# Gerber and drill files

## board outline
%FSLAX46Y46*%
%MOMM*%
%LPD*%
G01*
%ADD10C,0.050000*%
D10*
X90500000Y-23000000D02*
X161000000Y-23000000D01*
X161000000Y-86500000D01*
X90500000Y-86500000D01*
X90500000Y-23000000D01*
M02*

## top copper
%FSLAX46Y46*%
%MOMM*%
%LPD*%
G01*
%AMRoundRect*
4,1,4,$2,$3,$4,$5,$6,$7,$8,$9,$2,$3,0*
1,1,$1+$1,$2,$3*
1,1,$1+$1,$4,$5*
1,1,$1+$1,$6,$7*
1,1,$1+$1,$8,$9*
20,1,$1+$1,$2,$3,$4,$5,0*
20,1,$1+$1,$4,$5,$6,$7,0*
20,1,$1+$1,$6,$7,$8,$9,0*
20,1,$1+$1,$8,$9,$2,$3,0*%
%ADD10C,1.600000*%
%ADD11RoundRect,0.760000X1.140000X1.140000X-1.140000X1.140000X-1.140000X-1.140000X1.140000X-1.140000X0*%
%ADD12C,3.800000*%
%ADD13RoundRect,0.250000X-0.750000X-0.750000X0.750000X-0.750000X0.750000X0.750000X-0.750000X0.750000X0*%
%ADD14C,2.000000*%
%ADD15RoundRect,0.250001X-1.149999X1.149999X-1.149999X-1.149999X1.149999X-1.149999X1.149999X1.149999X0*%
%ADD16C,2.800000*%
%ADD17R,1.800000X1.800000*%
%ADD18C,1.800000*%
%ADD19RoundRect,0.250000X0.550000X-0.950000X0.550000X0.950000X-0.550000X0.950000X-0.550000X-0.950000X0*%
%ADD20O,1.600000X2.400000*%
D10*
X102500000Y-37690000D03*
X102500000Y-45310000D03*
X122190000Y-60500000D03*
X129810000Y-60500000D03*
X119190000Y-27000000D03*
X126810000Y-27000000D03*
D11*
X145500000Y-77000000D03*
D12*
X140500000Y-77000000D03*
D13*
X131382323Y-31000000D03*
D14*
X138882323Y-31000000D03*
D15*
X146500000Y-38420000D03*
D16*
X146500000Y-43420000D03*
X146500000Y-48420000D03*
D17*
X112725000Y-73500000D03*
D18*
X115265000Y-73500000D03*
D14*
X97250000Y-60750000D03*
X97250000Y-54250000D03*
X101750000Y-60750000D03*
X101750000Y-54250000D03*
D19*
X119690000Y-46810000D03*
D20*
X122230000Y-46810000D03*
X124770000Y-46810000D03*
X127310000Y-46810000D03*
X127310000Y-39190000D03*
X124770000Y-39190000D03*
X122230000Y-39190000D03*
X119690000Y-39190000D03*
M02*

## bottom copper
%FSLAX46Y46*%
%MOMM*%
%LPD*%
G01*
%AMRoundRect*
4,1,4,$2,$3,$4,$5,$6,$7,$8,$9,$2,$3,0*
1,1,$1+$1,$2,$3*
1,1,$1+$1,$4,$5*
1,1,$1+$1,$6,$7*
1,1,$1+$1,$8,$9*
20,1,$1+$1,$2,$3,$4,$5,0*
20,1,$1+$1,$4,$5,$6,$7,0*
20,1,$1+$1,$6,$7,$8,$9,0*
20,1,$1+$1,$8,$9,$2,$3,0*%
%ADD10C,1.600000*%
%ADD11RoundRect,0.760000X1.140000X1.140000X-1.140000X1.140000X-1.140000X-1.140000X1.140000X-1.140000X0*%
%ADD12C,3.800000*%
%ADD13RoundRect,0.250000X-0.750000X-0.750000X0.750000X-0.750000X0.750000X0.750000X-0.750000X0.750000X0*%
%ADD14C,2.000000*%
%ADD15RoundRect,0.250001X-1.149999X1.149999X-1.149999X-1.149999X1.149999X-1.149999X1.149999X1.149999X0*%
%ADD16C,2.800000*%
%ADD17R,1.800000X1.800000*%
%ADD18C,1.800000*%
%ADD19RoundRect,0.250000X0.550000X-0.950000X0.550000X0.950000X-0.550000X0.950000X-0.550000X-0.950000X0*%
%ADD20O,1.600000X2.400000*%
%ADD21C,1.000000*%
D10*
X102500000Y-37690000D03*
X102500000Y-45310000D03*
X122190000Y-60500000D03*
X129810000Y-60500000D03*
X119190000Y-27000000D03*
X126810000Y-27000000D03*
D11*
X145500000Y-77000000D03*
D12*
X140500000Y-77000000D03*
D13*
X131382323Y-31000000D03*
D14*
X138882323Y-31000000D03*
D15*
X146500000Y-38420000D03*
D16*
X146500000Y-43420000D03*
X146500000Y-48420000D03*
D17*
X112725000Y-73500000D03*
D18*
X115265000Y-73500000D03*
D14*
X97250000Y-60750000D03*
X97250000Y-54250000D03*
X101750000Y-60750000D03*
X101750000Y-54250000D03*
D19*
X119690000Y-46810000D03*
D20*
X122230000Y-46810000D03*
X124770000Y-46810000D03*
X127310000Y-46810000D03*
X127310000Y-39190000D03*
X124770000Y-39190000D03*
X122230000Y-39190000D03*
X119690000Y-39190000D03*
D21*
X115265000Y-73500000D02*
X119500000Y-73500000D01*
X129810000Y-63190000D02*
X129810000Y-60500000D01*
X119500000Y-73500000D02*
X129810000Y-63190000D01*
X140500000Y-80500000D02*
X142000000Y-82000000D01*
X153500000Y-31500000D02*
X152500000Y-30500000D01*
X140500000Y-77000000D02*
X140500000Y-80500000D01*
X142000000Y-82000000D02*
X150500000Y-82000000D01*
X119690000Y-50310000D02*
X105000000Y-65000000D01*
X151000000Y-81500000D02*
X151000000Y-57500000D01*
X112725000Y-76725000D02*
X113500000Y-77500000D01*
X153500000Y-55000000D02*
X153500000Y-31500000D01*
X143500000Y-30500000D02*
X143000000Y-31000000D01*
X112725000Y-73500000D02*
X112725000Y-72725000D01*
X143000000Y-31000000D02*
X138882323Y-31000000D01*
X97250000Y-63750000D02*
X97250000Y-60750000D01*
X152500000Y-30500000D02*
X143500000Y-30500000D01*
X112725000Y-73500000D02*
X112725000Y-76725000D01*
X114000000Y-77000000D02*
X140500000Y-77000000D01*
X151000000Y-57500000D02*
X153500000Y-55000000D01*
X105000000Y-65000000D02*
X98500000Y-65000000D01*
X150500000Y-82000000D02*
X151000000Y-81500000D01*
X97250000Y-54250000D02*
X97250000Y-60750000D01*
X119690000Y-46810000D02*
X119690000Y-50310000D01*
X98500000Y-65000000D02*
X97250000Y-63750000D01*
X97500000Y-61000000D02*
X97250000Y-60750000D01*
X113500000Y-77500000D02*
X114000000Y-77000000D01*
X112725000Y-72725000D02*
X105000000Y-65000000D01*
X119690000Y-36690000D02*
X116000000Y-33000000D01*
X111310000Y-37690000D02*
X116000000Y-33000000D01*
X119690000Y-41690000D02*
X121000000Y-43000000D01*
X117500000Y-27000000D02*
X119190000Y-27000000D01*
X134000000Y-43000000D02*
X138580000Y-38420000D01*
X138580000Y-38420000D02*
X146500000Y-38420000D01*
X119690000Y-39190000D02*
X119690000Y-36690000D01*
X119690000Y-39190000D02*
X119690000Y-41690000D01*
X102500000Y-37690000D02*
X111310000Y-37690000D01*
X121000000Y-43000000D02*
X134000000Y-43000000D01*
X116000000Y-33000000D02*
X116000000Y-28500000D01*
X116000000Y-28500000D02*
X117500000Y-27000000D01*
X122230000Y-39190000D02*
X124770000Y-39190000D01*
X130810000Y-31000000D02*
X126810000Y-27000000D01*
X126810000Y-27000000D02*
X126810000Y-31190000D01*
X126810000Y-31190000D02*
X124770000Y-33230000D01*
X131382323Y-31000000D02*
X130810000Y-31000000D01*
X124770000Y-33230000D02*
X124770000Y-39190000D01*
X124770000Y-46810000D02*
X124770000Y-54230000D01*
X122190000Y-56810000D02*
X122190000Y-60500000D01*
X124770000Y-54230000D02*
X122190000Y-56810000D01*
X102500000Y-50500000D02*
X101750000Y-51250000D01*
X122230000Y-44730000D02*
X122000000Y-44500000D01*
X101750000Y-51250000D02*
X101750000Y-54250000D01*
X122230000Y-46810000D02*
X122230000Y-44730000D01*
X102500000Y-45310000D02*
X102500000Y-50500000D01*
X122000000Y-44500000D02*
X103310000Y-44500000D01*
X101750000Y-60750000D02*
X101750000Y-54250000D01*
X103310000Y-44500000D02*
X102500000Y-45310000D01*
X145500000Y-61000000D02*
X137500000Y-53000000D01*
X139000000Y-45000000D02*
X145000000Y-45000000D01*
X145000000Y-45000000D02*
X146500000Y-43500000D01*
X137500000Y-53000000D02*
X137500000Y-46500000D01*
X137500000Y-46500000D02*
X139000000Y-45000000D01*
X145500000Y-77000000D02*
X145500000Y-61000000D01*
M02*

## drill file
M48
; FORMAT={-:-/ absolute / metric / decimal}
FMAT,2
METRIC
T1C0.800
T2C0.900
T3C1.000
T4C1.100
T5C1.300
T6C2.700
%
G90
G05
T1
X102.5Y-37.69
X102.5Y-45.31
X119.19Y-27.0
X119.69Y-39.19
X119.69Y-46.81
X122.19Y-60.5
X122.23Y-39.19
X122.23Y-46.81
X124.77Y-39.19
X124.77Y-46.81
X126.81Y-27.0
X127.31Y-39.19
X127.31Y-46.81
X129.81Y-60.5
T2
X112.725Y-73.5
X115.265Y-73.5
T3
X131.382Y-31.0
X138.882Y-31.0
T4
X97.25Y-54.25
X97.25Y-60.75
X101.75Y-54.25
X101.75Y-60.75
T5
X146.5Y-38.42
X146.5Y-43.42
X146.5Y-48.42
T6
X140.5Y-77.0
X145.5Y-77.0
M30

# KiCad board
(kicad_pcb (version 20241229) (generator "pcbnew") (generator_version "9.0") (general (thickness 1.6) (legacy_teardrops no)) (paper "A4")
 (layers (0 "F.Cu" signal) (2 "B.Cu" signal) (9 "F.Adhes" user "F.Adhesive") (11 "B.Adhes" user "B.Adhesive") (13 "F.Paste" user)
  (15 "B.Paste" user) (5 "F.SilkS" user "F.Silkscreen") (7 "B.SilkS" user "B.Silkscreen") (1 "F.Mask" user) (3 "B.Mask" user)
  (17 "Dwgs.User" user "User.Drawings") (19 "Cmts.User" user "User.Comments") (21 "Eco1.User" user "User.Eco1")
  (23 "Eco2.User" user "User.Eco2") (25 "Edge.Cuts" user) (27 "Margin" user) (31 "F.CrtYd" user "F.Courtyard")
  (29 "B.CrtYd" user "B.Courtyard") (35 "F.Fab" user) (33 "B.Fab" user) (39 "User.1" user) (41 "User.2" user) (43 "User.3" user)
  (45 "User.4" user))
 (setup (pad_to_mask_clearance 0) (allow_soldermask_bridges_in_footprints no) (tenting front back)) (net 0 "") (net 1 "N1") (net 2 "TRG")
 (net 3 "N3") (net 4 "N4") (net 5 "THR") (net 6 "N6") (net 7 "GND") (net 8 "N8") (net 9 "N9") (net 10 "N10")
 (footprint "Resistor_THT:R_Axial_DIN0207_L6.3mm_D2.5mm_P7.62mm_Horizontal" (layer "F.Cu") (at 102.5 37.69 -90)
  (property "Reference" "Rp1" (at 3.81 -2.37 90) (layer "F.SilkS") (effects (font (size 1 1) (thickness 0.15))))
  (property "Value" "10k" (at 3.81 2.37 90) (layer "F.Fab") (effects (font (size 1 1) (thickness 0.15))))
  (pad "1" thru_hole circle (at 0 0 270) (size 1.6 1.6) (drill 0.8) (layers "*.Cu" "*.Mask") (remove_unused_layers no) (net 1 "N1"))
  (pad "2" thru_hole circle (at 7.62 0 270) (size 1.6 1.6) (drill 0.8) (layers "*.Cu" "*.Mask") (remove_unused_layers no) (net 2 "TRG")))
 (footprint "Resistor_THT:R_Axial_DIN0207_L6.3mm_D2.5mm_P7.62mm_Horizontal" (layer "F.Cu") (at 122.19 60.5)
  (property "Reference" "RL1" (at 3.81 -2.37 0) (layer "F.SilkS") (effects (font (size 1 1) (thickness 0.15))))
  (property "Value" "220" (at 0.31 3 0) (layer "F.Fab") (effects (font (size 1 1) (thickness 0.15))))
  (pad "1" thru_hole circle (at 0 0) (size 1.6 1.6) (drill 0.8) (layers "*.Cu" "*.Mask") (remove_unused_layers no) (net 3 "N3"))
  (pad "2" thru_hole circle (at 7.62 0) (size 1.6 1.6) (drill 0.8) (layers "*.Cu" "*.Mask") (remove_unused_layers no) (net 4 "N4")))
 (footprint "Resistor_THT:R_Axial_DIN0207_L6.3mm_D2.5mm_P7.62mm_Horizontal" (layer "F.Cu") (at 119.19 27)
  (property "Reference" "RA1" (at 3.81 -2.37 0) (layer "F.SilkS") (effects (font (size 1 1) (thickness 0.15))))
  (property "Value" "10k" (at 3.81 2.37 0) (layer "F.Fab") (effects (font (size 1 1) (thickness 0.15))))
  (pad "1" thru_hole circle (at 0 0) (size 1.6 1.6) (drill 0.8) (layers "*.Cu" "*.Mask") (remove_unused_layers no) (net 1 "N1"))
  (pad "2" thru_hole circle (at 7.62 0) (size 1.6 1.6) (drill 0.8) (layers "*.Cu" "*.Mask") (remove_unused_layers no) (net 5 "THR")))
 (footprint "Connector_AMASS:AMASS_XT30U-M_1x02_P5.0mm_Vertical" (layer "F.Cu") (at 145.5 77 180)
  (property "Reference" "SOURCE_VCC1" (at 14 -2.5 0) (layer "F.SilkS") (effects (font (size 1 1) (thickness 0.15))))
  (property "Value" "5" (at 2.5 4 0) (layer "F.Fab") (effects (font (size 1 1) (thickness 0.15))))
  (pad "1" thru_hole roundrect (at 0 0 180) (size 3.8 3.8) (drill 2.7) (layers "*.Cu" "*.Mask") (remove_unused_layers no)
   (roundrect_rratio 0.2) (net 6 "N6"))
  (pad "2" thru_hole circle (at 5 0 180) (size 3.8 3.8) (drill 2.7) (layers "*.Cu" "*.Mask") (remove_unused_layers no) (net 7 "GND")))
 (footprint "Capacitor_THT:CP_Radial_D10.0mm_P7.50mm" (layer "F.Cu") (at 131.382323 31)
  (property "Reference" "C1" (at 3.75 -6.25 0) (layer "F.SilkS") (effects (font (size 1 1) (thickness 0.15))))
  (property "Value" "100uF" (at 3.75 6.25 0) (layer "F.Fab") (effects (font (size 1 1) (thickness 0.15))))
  (pad "1" thru_hole roundrect (at 0 0) (size 2 2) (drill 1) (layers "*.Cu" "*.Mask") (remove_unused_layers no) (roundrect_rratio 0.125)
   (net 5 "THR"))
  (pad "2" thru_hole circle (at 7.5 0) (size 2 2) (drill 1) (layers "*.Cu" "*.Mask") (remove_unused_layers no) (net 7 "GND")))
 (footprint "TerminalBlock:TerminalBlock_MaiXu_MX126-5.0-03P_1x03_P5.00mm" (layer "F.Cu") (at 146.5 38.42 -90)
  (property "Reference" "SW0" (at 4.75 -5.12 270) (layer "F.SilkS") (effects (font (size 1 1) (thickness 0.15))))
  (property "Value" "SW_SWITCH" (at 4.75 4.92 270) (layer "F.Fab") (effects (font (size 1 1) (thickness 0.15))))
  (pad "1" thru_hole roundrect (at 0 0 270) (size 2.8 2.8) (drill 1.3) (layers "*.Cu" "*.Mask") (remove_unused_layers no)
   (roundrect_rratio 0.089286) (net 1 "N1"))
  (pad "2" thru_hole circle (at 5 0 270) (size 2.8 2.8) (drill 1.3) (layers "*.Cu" "*.Mask") (remove_unused_layers no) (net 6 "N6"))
  (pad "3" thru_hole circle (at 10 0 270) (size 2.8 2.8) (drill 1.3) (layers "*.Cu" "*.Mask") (remove_unused_layers no) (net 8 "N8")))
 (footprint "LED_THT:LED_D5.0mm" (layer "F.Cu") (at 112.725 73.5)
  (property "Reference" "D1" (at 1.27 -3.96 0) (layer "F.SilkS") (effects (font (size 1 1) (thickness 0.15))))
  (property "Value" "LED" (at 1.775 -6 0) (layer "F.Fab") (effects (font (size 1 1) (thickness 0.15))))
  (pad "1" thru_hole rect (at 0 0) (size 1.8 1.8) (drill 0.9) (layers "*.Cu" "*.Mask") (remove_unused_layers no) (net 7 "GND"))
  (pad "2" thru_hole circle (at 2.54 0) (size 1.8 1.8) (drill 0.9) (layers "*.Cu" "*.Mask") (remove_unused_layers no) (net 4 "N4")))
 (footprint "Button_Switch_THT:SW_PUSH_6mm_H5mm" (layer "F.Cu") (at 97.25 60.75 90)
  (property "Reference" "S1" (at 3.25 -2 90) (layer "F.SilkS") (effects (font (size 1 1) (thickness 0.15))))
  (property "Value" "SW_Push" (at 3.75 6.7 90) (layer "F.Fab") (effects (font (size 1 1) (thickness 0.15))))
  (pad "1" thru_hole circle (at 0 0 180) (size 2 2) (drill 1.1) (layers "*.Cu" "*.Mask") (remove_unused_layers no) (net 7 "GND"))
  (pad "1" thru_hole circle (at 6.5 0 180) (size 2 2) (drill 1.1) (layers "*.Cu" "*.Mask") (remove_unused_layers no) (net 7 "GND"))
  (pad "2" thru_hole circle (at 0 4.5 180) (size 2 2) (drill 1.1) (layers "*.Cu" "*.Mask") (remove_unused_layers no) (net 2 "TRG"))
  (pad "2" thru_hole circle (at 6.5 4.5 180) (size 2 2) (drill 1.1) (layers "*.Cu" "*.Mask") (remove_unused_layers no) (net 2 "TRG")))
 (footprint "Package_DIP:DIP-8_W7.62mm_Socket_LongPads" (layer "F.Cu") (at 119.69 46.81 90)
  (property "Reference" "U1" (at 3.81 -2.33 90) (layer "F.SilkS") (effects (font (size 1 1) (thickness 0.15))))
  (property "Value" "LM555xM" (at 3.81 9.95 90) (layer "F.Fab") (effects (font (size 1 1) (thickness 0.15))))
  (pad "1" thru_hole roundrect (at 0 0 90) (size 2.4 1.6) (drill 0.8) (layers "*.Cu" "*.Mask") (remove_unused_layers no)
   (roundrect_rratio 0.15625) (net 7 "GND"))
  (pad "2" thru_hole oval (at 0 2.54 90) (size 2.4 1.6) (drill 0.8) (layers "*.Cu" "*.Mask") (remove_unused_layers no) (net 2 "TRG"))
  (pad "3" thru_hole oval (at 0 5.08 90) (size 2.4 1.6) (drill 0.8) (layers "*.Cu" "*.Mask") (remove_unused_layers no) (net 3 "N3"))
  (pad "4" thru_hole oval (at 0 7.62 90) (size 2.4 1.6) (drill 0.8) (layers "*.Cu" "*.Mask") (remove_unused_layers no) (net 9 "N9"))
  (pad "5" thru_hole oval (at 7.62 7.62 90) (size 2.4 1.6) (drill 0.8) (layers "*.Cu" "*.Mask") (remove_unused_layers no) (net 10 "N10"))
  (pad "6" thru_hole oval (at 7.62 5.08 90) (size 2.4 1.6) (drill 0.8) (layers "*.Cu" "*.Mask") (remove_unused_layers no) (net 5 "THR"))
  (pad "7" thru_hole oval (at 7.62 2.54 90) (size 2.4 1.6) (drill 0.8) (layers "*.Cu" "*.Mask") (remove_unused_layers no) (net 5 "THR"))
  (pad "8" thru_hole oval (at 7.62 0 90) (size 2.4 1.6) (drill 0.8) (layers "*.Cu" "*.Mask") (remove_unused_layers no) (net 1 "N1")))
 (gr_rect (start 90.5 23) (end 161 86.5) (stroke (width 0.05) (type default)) (fill no) (layer "Edge.Cuts"))
 (segment (start 115.265 73.5) (end 119.5 73.5) (width 1) (layer "B.Cu") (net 4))
 (segment (start 129.81 63.19) (end 129.81 60.5) (width 1) (layer "B.Cu") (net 4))
 (segment (start 119.5 73.5) (end 129.81 63.19) (width 1) (layer "B.Cu") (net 4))
 (segment (start 140.5 80.5) (end 142 82) (width 1) (layer "B.Cu") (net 7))
 (segment (start 153.5 31.5) (end 152.5 30.5) (width 1) (layer "B.Cu") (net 7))
 (segment (start 140.5 77) (end 140.5 80.5) (width 1) (layer "B.Cu") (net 7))
 (segment (start 142 82) (end 150.5 82) (width 1) (layer "B.Cu") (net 7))
 (segment (start 119.69 50.31) (end 105 65) (width 1) (layer "B.Cu") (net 7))
 (segment (start 151 81.5) (end 151 57.5) (width 1) (layer "B.Cu") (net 7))
 (segment (start 112.725 76.725) (end 113.5 77.5) (width 1) (layer "B.Cu") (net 7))
 (segment (start 153.5 55) (end 153.5 31.5) (width 1) (layer "B.Cu") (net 7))
 (segment (start 143.5 30.5) (end 143 31) (width 1) (layer "B.Cu") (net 7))
 (segment (start 112.725 73.5) (end 112.725 72.725) (width 1) (layer "B.Cu") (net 7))
 (segment (start 143 31) (end 138.882323 31) (width 1) (layer "B.Cu") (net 7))
 (segment (start 97.25 63.75) (end 97.25 60.75) (width 1) (layer "B.Cu") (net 7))
 (segment (start 152.5 30.5) (end 143.5 30.5) (width 1) (layer "B.Cu") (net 7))
 (segment (start 112.725 73.5) (end 112.725 76.725) (width 1) (layer "B.Cu") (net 7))
 (segment (start 114 77) (end 140.5 77) (width 1) (layer "B.Cu") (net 7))
 (segment (start 151 57.5) (end 153.5 55) (width 1) (layer "B.Cu") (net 7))
 (segment (start 105 65) (end 98.5 65) (width 1) (layer "B.Cu") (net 7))
 (segment (start 150.5 82) (end 151 81.5) (width 1) (layer "B.Cu") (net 7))
 (segment (start 97.25 54.25) (end 97.25 60.75) (width 1) (layer "B.Cu") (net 7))
 (segment (start 119.69 46.81) (end 119.69 50.31) (width 1) (layer "B.Cu") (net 7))
 (segment (start 98.5 65) (end 97.25 63.75) (width 1) (layer "B.Cu") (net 7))
 (segment (start 97.5 61) (end 97.25 60.75) (width 1) (layer "B.Cu") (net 7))
 (segment (start 113.5 77.5) (end 114 77) (width 1) (layer "B.Cu") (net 7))
 (segment (start 112.725 72.725) (end 105 65) (width 1) (layer "B.Cu") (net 7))
 (segment (start 119.69 36.69) (end 116 33) (width 1) (layer "B.Cu") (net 1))
 (segment (start 111.31 37.69) (end 116 33) (width 1) (layer "B.Cu") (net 1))
 (segment (start 119.69 41.69) (end 121 43) (width 1) (layer "B.Cu") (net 1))
 (segment (start 117.5 27) (end 119.19 27) (width 1) (layer "B.Cu") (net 1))
 (segment (start 134 43) (end 138.58 38.42) (width 1) (layer "B.Cu") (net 1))
 (segment (start 138.58 38.42) (end 146.5 38.42) (width 1) (layer "B.Cu") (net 1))
 (segment (start 119.69 39.19) (end 119.69 36.69) (width 1) (layer "B.Cu") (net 1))
 (segment (start 119.69 39.19) (end 119.69 41.69) (width 1) (layer "B.Cu") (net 1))
 (segment (start 102.5 37.69) (end 111.31 37.69) (width 1) (layer "B.Cu") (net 1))
 (segment (start 121 43) (end 134 43) (width 1) (layer "B.Cu") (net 1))
 (segment (start 116 33) (end 116 28.5) (width 1) (layer "B.Cu") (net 1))
 (segment (start 116 28.5) (end 117.5 27) (width 1) (layer "B.Cu") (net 1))
 (segment (start 122.23 39.19) (end 124.77 39.19) (width 1) (layer "B.Cu") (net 5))
 (segment (start 130.81 31) (end 126.81 27) (width 1) (layer "B.Cu") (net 5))
 (segment (start 126.81 27) (end 126.81 31.19) (width 1) (layer "B.Cu") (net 5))
 (segment (start 126.81 31.19) (end 124.77 33.23) (width 1) (layer "B.Cu") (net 5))
 (segment (start 131.382323 31) (end 130.81 31) (width 1) (layer "B.Cu") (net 5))
 (segment (start 124.77 33.23) (end 124.77 39.19) (width 1) (layer "B.Cu") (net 5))
 (segment (start 124.77 46.81) (end 124.77 54.23) (width 1) (layer "B.Cu") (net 3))
 (segment (start 122.19 56.81) (end 122.19 60.5) (width 1) (layer "B.Cu") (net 3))
 (segment (start 124.77 54.23) (end 122.19 56.81) (width 1) (layer "B.Cu") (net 3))
 (segment (start 102.5 50.5) (end 101.75 51.25) (width 1) (layer "B.Cu") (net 2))
 (segment (start 122.23 44.73) (end 122 44.5) (width 1) (layer "B.Cu") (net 2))
 (segment (start 101.75 51.25) (end 101.75 54.25) (width 1) (layer "B.Cu") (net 2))
 (segment (start 122.23 46.81) (end 122.23 44.73) (width 1) (layer "B.Cu") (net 2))
 (segment (start 102.5 45.31) (end 102.5 50.5) (width 1) (layer "B.Cu") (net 2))
 (segment (start 122 44.5) (end 103.31 44.5) (width 1) (layer "B.Cu") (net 2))
 (segment (start 101.75 60.75) (end 101.75 54.25) (width 1) (layer "B.Cu") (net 2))
 (segment (start 103.31 44.5) (end 102.5 45.31) (width 1) (layer "B.Cu") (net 2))
 (segment (start 145.5 61) (end 137.5 53) (width 1) (layer "B.Cu") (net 6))
 (segment (start 139 45) (end 145 45) (width 1) (layer "B.Cu") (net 6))
 (segment (start 145 45) (end 146.5 43.5) (width 1) (layer "B.Cu") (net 6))
 (segment (start 137.5 53) (end 137.5 46.5) (width 1) (layer "B.Cu") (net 6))
 (segment (start 137.5 46.5) (end 139 45) (width 1) (layer "B.Cu") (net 6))
 (segment (start 145.5 77) (end 145.5 61) (width 1) (layer "B.Cu") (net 6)))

